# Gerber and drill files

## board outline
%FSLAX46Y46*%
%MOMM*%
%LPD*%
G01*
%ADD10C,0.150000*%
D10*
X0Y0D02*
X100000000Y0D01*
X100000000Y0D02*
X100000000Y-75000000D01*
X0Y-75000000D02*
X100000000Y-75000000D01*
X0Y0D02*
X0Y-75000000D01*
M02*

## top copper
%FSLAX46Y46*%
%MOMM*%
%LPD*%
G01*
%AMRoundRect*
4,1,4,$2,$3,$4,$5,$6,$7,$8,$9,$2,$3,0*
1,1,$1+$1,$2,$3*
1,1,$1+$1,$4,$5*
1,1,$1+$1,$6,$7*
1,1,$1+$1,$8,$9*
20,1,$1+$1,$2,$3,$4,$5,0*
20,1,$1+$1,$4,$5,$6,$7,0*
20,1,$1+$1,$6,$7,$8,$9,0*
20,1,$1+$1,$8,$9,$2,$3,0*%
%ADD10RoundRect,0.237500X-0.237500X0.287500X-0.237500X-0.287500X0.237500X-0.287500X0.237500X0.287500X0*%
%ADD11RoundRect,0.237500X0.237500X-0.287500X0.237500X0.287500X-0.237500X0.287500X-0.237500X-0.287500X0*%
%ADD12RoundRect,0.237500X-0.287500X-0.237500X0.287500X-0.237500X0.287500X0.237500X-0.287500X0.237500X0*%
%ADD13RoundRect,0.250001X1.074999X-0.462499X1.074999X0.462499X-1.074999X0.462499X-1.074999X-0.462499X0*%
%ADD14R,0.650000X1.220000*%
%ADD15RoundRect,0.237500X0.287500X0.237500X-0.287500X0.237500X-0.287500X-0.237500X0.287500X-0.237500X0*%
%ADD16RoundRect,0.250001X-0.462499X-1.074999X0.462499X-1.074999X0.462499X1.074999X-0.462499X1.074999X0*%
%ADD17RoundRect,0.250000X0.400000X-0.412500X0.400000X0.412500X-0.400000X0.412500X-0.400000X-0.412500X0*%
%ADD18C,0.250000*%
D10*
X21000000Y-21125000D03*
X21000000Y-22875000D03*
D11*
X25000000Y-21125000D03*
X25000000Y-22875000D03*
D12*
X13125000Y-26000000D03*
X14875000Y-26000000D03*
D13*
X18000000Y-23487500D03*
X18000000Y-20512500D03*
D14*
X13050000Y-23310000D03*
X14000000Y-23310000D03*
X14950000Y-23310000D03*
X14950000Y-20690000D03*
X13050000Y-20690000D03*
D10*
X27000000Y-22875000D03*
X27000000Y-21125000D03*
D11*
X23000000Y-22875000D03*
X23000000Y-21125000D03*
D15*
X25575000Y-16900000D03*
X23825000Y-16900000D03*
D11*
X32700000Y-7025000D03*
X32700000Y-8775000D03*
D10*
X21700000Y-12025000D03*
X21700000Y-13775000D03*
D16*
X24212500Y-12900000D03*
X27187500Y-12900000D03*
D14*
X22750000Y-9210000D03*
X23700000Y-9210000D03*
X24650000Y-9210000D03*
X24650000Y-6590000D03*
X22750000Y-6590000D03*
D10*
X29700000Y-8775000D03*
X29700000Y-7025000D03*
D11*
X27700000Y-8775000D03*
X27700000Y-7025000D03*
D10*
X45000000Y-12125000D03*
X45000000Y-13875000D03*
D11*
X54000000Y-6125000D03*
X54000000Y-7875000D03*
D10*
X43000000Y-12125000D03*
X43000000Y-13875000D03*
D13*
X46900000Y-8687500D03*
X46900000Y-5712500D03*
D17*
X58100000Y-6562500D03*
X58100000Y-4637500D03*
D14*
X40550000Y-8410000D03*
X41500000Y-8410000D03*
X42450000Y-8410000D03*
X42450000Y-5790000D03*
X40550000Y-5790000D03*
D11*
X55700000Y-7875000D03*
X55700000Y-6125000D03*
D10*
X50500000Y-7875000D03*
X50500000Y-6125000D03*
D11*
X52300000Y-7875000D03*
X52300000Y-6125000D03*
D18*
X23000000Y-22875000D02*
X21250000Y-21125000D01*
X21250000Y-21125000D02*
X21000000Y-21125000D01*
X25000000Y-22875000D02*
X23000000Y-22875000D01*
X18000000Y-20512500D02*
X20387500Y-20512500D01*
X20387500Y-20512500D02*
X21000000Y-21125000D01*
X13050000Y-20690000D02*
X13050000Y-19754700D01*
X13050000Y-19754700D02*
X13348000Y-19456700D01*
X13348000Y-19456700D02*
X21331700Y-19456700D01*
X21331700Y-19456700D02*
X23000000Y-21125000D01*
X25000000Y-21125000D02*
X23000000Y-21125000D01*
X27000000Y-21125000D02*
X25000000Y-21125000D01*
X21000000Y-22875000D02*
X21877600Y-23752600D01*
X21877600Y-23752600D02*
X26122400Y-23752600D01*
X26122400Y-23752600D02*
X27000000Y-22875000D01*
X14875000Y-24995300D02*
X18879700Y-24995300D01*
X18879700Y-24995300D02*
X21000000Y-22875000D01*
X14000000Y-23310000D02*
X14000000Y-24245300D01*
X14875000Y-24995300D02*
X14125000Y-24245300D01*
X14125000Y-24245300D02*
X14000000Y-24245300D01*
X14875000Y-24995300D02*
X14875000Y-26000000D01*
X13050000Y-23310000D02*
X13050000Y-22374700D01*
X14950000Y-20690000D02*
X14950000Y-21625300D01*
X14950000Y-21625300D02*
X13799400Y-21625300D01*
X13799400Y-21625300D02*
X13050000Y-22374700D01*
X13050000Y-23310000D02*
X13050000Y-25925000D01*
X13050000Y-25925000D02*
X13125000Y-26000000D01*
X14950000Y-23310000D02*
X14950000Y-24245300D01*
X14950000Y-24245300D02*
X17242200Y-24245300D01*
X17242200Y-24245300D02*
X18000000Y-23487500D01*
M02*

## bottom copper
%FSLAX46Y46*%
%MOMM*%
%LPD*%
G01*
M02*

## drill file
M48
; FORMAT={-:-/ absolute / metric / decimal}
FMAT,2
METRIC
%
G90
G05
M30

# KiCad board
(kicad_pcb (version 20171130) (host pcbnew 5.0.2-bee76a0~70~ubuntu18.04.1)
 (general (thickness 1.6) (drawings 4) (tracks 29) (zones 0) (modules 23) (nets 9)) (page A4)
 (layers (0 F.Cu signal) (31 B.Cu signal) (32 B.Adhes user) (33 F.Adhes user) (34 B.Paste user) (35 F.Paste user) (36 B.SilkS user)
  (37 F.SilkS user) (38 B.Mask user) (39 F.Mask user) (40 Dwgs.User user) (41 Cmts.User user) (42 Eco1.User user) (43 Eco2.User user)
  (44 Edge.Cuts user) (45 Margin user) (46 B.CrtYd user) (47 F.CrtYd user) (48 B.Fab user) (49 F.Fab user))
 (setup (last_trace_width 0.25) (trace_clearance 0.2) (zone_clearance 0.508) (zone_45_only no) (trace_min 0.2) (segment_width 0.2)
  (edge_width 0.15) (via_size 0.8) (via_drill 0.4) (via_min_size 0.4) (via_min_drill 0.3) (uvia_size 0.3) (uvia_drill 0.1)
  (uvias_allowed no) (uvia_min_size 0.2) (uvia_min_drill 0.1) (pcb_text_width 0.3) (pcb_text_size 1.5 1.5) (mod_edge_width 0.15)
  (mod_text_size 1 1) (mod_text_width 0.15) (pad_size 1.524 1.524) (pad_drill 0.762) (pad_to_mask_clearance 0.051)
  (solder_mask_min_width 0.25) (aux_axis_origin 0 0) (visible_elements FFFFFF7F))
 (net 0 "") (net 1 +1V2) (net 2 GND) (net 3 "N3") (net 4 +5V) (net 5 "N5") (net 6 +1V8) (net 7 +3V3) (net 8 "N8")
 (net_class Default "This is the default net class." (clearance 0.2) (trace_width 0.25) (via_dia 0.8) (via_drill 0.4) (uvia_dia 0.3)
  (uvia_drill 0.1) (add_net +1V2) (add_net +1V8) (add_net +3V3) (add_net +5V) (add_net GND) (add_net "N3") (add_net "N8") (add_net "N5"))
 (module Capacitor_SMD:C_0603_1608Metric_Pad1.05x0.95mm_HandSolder (layer F.Cu) (at 21 22 270)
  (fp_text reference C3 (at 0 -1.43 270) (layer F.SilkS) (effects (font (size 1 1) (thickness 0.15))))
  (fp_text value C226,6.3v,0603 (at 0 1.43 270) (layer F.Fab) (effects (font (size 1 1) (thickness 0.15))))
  (pad 1 smd roundrect (at -0.875 0 270) (size 1.05 0.95) (layers F.Cu F.Paste F.Mask) (roundrect_rratio 0.25) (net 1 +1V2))
  (pad 2 smd roundrect (at 0.875 0 270) (size 1.05 0.95) (layers F.Cu F.Paste F.Mask) (roundrect_rratio 0.25) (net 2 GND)))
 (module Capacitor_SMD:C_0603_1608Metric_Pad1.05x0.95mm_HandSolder (layer F.Cu) (at 25 22 90)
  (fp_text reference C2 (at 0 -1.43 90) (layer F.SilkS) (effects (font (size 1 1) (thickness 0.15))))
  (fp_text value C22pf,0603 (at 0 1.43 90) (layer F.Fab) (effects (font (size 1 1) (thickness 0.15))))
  (pad 2 smd roundrect (at 0.875 0 90) (size 1.05 0.95) (layers F.Cu F.Paste F.Mask) (roundrect_rratio 0.25) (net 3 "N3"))
  (pad 1 smd roundrect (at -0.875 0 90) (size 1.05 0.95) (layers F.Cu F.Paste F.Mask) (roundrect_rratio 0.25) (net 1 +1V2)))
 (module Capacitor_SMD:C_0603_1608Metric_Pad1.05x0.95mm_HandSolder (layer F.Cu) (at 14 26)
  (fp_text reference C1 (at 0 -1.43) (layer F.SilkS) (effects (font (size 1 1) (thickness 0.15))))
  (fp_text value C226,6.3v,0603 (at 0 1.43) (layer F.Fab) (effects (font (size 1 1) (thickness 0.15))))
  (pad 1 smd roundrect (at -0.875 0) (size 1.05 0.95) (layers F.Cu F.Paste F.Mask) (roundrect_rratio 0.25) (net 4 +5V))
  (pad 2 smd roundrect (at 0.875 0) (size 1.05 0.95) (layers F.Cu F.Paste F.Mask) (roundrect_rratio 0.25) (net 2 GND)))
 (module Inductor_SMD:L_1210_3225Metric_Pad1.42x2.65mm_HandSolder (layer F.Cu) (at 18 22 90)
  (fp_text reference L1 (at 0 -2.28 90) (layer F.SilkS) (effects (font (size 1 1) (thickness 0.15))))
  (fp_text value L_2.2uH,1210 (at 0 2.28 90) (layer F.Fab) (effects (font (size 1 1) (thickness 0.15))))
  (pad 1 smd roundrect (at -1.4875 0 90) (size 1.425 2.65) (layers F.Cu F.Paste F.Mask) (roundrect_rratio 0.175439) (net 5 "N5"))
  (pad 2 smd roundrect (at 1.4875 0 90) (size 1.425 2.65) (layers F.Cu F.Paste F.Mask) (roundrect_rratio 0.175439) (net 1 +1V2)))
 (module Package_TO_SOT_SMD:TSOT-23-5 (layer F.Cu) (at 14 22 90)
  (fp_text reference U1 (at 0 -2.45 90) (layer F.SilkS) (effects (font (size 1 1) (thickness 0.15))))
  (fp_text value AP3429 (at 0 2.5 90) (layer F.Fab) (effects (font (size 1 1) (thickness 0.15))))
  (pad 1 smd rect (at -1.31 -0.95 90) (size 1.22 0.65) (layers F.Cu F.Paste F.Mask) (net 4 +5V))
  (pad 2 smd rect (at -1.31 0 90) (size 1.22 0.65) (layers F.Cu F.Paste F.Mask) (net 2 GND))
  (pad 3 smd rect (at -1.31 0.95 90) (size 1.22 0.65) (layers F.Cu F.Paste F.Mask) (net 5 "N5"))
  (pad 4 smd rect (at 1.31 0.95 90) (size 1.22 0.65) (layers F.Cu F.Paste F.Mask) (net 4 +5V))
  (pad 5 smd rect (at 1.31 -0.95 90) (size 1.22 0.65) (layers F.Cu F.Paste F.Mask) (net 3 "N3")))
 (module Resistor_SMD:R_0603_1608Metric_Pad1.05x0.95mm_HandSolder (layer F.Cu) (at 27 22 270)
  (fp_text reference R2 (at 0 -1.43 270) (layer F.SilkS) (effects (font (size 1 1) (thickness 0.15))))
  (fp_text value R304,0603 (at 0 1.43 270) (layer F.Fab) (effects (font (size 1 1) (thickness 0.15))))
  (pad 2 smd roundrect (at 0.875 0 270) (size 1.05 0.95) (layers F.Cu F.Paste F.Mask) (roundrect_rratio 0.25) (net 2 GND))
  (pad 1 smd roundrect (at -0.875 0 270) (size 1.05 0.95) (layers F.Cu F.Paste F.Mask) (roundrect_rratio 0.25) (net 3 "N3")))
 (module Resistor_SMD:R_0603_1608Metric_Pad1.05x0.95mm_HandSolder (layer F.Cu) (at 23 22 90)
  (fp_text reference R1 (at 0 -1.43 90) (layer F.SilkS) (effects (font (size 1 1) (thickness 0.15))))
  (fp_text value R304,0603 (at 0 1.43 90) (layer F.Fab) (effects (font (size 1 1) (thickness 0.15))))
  (pad 1 smd roundrect (at -0.875 0 90) (size 1.05 0.95) (layers F.Cu F.Paste F.Mask) (roundrect_rratio 0.25) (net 1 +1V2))
  (pad 2 smd roundrect (at 0.875 0 90) (size 1.05 0.95) (layers F.Cu F.Paste F.Mask) (roundrect_rratio 0.25) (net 3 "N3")))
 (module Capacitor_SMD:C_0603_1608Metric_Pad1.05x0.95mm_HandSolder (layer F.Cu) (at 24.7 16.9 180)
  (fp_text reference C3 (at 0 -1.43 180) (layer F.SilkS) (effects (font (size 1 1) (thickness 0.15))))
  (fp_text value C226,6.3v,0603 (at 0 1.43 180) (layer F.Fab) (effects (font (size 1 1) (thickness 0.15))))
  (pad 1 smd roundrect (at -0.875 0 180) (size 1.05 0.95) (layers F.Cu F.Paste F.Mask) (roundrect_rratio 0.25) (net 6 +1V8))
  (pad 2 smd roundrect (at 0.875 0 180) (size 1.05 0.95) (layers F.Cu F.Paste F.Mask) (roundrect_rratio 0.25) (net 2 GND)))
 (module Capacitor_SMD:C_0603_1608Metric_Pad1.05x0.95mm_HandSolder (layer F.Cu) (at 32.7 7.9 90)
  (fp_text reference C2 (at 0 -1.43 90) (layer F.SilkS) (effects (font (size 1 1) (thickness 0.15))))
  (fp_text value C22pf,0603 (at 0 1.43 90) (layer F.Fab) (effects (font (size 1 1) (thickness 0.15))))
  (pad 2 smd roundrect (at 0.875 0 90) (size 1.05 0.95) (layers F.Cu F.Paste F.Mask) (roundrect_rratio 0.25) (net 3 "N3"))
  (pad 1 smd roundrect (at -0.875 0 90) (size 1.05 0.95) (layers F.Cu F.Paste F.Mask) (roundrect_rratio 0.25) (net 6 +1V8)))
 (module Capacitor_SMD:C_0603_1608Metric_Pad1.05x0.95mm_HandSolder (layer F.Cu) (at 21.7 12.9 270)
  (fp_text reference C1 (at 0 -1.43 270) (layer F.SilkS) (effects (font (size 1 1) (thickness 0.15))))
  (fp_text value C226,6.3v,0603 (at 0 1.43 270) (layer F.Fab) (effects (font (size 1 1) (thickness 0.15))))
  (pad 1 smd roundrect (at -0.875 0 270) (size 1.05 0.95) (layers F.Cu F.Paste F.Mask) (roundrect_rratio 0.25) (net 4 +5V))
  (pad 2 smd roundrect (at 0.875 0 270) (size 1.05 0.95) (layers F.Cu F.Paste F.Mask) (roundrect_rratio 0.25) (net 2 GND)))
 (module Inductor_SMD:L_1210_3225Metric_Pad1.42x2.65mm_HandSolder (layer F.Cu) (at 25.7 12.9)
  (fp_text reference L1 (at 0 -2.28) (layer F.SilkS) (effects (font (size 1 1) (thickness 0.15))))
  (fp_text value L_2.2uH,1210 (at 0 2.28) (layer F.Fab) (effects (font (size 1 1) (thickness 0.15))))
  (pad 1 smd roundrect (at -1.4875 0) (size 1.425 2.65) (layers F.Cu F.Paste F.Mask) (roundrect_rratio 0.175439) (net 5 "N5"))
  (pad 2 smd roundrect (at 1.4875 0) (size 1.425 2.65) (layers F.Cu F.Paste F.Mask) (roundrect_rratio 0.175439) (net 6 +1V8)))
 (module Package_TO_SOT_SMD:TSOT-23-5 (layer F.Cu) (at 23.7 7.9 90)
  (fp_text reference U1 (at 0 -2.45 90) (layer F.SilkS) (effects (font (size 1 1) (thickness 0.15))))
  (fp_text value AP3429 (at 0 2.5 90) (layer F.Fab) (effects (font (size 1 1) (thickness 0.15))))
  (pad 1 smd rect (at -1.31 -0.95 90) (size 1.22 0.65) (layers F.Cu F.Paste F.Mask) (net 4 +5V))
  (pad 2 smd rect (at -1.31 0 90) (size 1.22 0.65) (layers F.Cu F.Paste F.Mask) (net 2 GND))
  (pad 3 smd rect (at -1.31 0.95 90) (size 1.22 0.65) (layers F.Cu F.Paste F.Mask) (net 5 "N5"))
  (pad 4 smd rect (at 1.31 0.95 90) (size 1.22 0.65) (layers F.Cu F.Paste F.Mask) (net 4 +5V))
  (pad 5 smd rect (at 1.31 -0.95 90) (size 1.22 0.65) (layers F.Cu F.Paste F.Mask) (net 3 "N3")))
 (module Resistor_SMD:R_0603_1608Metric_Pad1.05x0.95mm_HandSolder (layer F.Cu) (at 29.7 7.9 270)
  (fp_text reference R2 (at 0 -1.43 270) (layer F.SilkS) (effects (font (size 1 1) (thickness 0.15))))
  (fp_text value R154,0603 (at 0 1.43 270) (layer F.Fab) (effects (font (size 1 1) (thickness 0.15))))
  (pad 2 smd roundrect (at 0.875 0 270) (size 1.05 0.95) (layers F.Cu F.Paste F.Mask) (roundrect_rratio 0.25) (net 2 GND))
  (pad 1 smd roundrect (at -0.875 0 270) (size 1.05 0.95) (layers F.Cu F.Paste F.Mask) (roundrect_rratio 0.25) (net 3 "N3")))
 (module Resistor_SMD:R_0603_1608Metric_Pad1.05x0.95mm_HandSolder (layer F.Cu) (at 27.7 7.9 90)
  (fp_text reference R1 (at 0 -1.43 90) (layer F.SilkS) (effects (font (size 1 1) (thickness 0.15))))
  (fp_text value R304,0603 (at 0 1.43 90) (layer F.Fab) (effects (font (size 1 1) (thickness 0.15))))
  (pad 1 smd roundrect (at -0.875 0 90) (size 1.05 0.95) (layers F.Cu F.Paste F.Mask) (roundrect_rratio 0.25) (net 6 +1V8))
  (pad 2 smd roundrect (at 0.875 0 90) (size 1.05 0.95) (layers F.Cu F.Paste F.Mask) (roundrect_rratio 0.25) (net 3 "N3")))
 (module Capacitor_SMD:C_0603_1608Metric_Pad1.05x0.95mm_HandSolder (layer F.Cu) (at 45 13 270)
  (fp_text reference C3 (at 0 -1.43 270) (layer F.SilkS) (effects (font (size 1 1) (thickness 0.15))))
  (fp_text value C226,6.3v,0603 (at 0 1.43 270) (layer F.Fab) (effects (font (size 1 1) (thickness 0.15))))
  (pad 1 smd roundrect (at -0.875 0 270) (size 1.05 0.95) (layers F.Cu F.Paste F.Mask) (roundrect_rratio 0.25) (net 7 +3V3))
  (pad 2 smd roundrect (at 0.875 0 270) (size 1.05 0.95) (layers F.Cu F.Paste F.Mask) (roundrect_rratio 0.25) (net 2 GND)))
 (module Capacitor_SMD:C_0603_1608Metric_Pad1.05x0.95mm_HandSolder (layer F.Cu) (at 54 7 90)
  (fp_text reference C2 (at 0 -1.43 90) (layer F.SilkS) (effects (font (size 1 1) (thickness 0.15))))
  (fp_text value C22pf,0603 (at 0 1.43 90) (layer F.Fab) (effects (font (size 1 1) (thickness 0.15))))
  (pad 2 smd roundrect (at 0.875 0 90) (size 1.05 0.95) (layers F.Cu F.Paste F.Mask) (roundrect_rratio 0.25) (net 3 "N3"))
  (pad 1 smd roundrect (at -0.875 0 90) (size 1.05 0.95) (layers F.Cu F.Paste F.Mask) (roundrect_rratio 0.25) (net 7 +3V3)))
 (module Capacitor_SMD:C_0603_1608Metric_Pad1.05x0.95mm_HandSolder (layer F.Cu) (at 43 13 270)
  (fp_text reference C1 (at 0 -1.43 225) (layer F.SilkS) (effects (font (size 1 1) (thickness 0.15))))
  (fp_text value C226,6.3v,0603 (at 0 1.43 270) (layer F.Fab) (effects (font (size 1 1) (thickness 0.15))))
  (pad 1 smd roundrect (at -0.875 0 270) (size 1.05 0.95) (layers F.Cu F.Paste F.Mask) (roundrect_rratio 0.25) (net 4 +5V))
  (pad 2 smd roundrect (at 0.875 0 270) (size 1.05 0.95) (layers F.Cu F.Paste F.Mask) (roundrect_rratio 0.25) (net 2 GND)))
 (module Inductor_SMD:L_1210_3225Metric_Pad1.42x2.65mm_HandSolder (layer F.Cu) (at 46.9 7.2 90)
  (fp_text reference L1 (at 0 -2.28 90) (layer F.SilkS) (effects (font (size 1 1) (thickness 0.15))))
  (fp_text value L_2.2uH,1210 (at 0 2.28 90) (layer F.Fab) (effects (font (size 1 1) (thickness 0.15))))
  (pad 1 smd roundrect (at -1.4875 0 90) (size 1.425 2.65) (layers F.Cu F.Paste F.Mask) (roundrect_rratio 0.175439) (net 5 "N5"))
  (pad 2 smd roundrect (at 1.4875 0 90) (size 1.425 2.65) (layers F.Cu F.Paste F.Mask) (roundrect_rratio 0.175439) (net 7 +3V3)))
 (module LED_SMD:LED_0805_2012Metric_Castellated (layer F.Cu) (at 58.1 5.6 90)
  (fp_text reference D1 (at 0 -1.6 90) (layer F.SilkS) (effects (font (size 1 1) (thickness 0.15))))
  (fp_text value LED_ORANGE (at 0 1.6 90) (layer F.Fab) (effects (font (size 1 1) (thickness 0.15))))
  (pad 1 smd roundrect (at -0.9625 0 90) (size 1.325 1.3) (layers F.Cu F.Paste F.Mask) (roundrect_rratio 0.192308) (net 2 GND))
  (pad 2 smd roundrect (at 0.9625 0 90) (size 1.325 1.3) (layers F.Cu F.Paste F.Mask) (roundrect_rratio 0.192308) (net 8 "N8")))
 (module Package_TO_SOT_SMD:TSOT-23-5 (layer F.Cu) (at 41.5 7.1 90)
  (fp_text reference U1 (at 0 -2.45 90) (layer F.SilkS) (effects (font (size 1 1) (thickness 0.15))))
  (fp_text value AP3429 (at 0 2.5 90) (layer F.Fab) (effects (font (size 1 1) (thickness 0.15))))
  (pad 1 smd rect (at -1.31 -0.95 90) (size 1.22 0.65) (layers F.Cu F.Paste F.Mask) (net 4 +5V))
  (pad 2 smd rect (at -1.31 0 90) (size 1.22 0.65) (layers F.Cu F.Paste F.Mask) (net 2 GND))
  (pad 3 smd rect (at -1.31 0.95 90) (size 1.22 0.65) (layers F.Cu F.Paste F.Mask) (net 5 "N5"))
  (pad 4 smd rect (at 1.31 0.95 90) (size 1.22 0.65) (layers F.Cu F.Paste F.Mask) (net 4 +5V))
  (pad 5 smd rect (at 1.31 -0.95 90) (size 1.22 0.65) (layers F.Cu F.Paste F.Mask) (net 3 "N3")))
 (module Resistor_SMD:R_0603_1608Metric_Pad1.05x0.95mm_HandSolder (layer F.Cu) (at 55.7 7 90)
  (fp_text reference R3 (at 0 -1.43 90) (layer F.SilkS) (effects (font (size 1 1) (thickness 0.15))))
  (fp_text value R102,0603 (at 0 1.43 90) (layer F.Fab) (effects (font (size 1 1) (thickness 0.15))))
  (pad 1 smd roundrect (at -0.875 0 90) (size 1.05 0.95) (layers F.Cu F.Paste F.Mask) (roundrect_rratio 0.25) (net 7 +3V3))
  (pad 2 smd roundrect (at 0.875 0 90) (size 1.05 0.95) (layers F.Cu F.Paste F.Mask) (roundrect_rratio 0.25) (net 8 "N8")))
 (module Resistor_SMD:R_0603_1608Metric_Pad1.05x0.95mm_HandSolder (layer F.Cu) (at 50.5 7 270)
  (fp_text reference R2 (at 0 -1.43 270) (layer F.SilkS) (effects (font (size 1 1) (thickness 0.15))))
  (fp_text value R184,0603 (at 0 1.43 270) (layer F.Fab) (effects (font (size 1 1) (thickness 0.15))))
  (pad 2 smd roundrect (at 0.875 0 270) (size 1.05 0.95) (layers F.Cu F.Paste F.Mask) (roundrect_rratio 0.25) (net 2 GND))
  (pad 1 smd roundrect (at -0.875 0 270) (size 1.05 0.95) (layers F.Cu F.Paste F.Mask) (roundrect_rratio 0.25) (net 3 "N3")))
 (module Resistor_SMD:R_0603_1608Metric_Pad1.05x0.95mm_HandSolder (layer F.Cu) (at 52.3 7 90)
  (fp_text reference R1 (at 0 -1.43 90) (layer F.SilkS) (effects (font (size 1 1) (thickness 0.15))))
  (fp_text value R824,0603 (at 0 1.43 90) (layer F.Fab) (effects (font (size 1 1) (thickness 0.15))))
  (pad 1 smd roundrect (at -0.875 0 90) (size 1.05 0.95) (layers F.Cu F.Paste F.Mask) (roundrect_rratio 0.25) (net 7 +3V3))
  (pad 2 smd roundrect (at 0.875 0 90) (size 1.05 0.95) (layers F.Cu F.Paste F.Mask) (roundrect_rratio 0.25) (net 3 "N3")))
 (gr_line (start 0 0) (end 100 0) (layer Edge.Cuts) (width 0.15))
 (gr_line (start 100 0) (end 100 75) (layer Edge.Cuts) (width 0.15))
 (gr_line (start 0 75) (end 100 75) (layer Edge.Cuts) (width 0.15))
 (gr_line (start 0 0) (end 0 75) (layer Edge.Cuts) (width 0.15))
 (segment (start 23 22.875) (end 21.25 21.125) (width 0.25) (layer F.Cu) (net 1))
 (segment (start 21.25 21.125) (end 21 21.125) (width 0.25) (layer F.Cu) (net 1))
 (segment (start 25 22.875) (end 23 22.875) (width 0.25) (layer F.Cu) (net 1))
 (segment (start 18 20.5125) (end 20.3875 20.5125) (width 0.25) (layer F.Cu) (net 1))
 (segment (start 20.3875 20.5125) (end 21 21.125) (width 0.25) (layer F.Cu) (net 1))
 (segment (start 13.05 20.69) (end 13.05 19.7547) (width 0.25) (layer F.Cu) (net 3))
 (segment (start 13.05 19.7547) (end 13.348 19.4567) (width 0.25) (layer F.Cu) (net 3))
 (segment (start 13.348 19.4567) (end 21.3317 19.4567) (width 0.25) (layer F.Cu) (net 3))
 (segment (start 21.3317 19.4567) (end 23 21.125) (width 0.25) (layer F.Cu) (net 3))
 (segment (start 25 21.125) (end 23 21.125) (width 0.25) (layer F.Cu) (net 3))
 (segment (start 27 21.125) (end 25 21.125) (width 0.25) (layer F.Cu) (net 3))
 (segment (start 21 22.875) (end 21.8776 23.7526) (width 0.25) (layer F.Cu) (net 2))
 (segment (start 21.8776 23.7526) (end 26.1224 23.7526) (width 0.25) (layer F.Cu) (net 2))
 (segment (start 26.1224 23.7526) (end 27 22.875) (width 0.25) (layer F.Cu) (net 2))
 (segment (start 14.875 24.9953) (end 18.8797 24.9953) (width 0.25) (layer F.Cu) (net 2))
 (segment (start 18.8797 24.9953) (end 21 22.875) (width 0.25) (layer F.Cu) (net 2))
 (segment (start 14 23.31) (end 14 24.2453) (width 0.25) (layer F.Cu) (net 2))
 (segment (start 14.875 24.9953) (end 14.125 24.2453) (width 0.25) (layer F.Cu) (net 2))
 (segment (start 14.125 24.2453) (end 14 24.2453) (width 0.25) (layer F.Cu) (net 2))
 (segment (start 14.875 24.9953) (end 14.875 26) (width 0.25) (layer F.Cu) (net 2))
 (segment (start 13.05 23.31) (end 13.05 22.3747) (width 0.25) (layer F.Cu) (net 4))
 (segment (start 14.95 20.69) (end 14.95 21.6253) (width 0.25) (layer F.Cu) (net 4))
 (segment (start 14.95 21.6253) (end 13.7994 21.6253) (width 0.25) (layer F.Cu) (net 4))
 (segment (start 13.7994 21.6253) (end 13.05 22.3747) (width 0.25) (layer F.Cu) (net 4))
 (segment (start 13.05 23.31) (end 13.05 25.925) (width 0.25) (layer F.Cu) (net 4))
 (segment (start 13.05 25.925) (end 13.125 26) (width 0.25) (layer F.Cu) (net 4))
 (segment (start 14.95 23.31) (end 14.95 24.2453) (width 0.25) (layer F.Cu) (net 5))
 (segment (start 14.95 24.2453) (end 17.2422 24.2453) (width 0.25) (layer F.Cu) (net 5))
 (segment (start 17.2422 24.2453) (end 18 23.4875) (width 0.25) (layer F.Cu) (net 5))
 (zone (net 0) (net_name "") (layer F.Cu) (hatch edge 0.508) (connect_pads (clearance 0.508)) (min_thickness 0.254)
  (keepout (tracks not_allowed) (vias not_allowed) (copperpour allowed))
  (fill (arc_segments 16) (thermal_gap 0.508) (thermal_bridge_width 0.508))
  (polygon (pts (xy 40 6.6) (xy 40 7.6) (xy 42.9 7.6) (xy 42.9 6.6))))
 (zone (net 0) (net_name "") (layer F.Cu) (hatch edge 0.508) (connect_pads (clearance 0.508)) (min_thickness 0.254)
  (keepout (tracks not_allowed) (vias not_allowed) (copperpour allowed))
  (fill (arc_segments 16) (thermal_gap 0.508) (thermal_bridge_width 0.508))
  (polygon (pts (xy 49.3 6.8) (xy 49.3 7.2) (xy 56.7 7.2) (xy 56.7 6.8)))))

